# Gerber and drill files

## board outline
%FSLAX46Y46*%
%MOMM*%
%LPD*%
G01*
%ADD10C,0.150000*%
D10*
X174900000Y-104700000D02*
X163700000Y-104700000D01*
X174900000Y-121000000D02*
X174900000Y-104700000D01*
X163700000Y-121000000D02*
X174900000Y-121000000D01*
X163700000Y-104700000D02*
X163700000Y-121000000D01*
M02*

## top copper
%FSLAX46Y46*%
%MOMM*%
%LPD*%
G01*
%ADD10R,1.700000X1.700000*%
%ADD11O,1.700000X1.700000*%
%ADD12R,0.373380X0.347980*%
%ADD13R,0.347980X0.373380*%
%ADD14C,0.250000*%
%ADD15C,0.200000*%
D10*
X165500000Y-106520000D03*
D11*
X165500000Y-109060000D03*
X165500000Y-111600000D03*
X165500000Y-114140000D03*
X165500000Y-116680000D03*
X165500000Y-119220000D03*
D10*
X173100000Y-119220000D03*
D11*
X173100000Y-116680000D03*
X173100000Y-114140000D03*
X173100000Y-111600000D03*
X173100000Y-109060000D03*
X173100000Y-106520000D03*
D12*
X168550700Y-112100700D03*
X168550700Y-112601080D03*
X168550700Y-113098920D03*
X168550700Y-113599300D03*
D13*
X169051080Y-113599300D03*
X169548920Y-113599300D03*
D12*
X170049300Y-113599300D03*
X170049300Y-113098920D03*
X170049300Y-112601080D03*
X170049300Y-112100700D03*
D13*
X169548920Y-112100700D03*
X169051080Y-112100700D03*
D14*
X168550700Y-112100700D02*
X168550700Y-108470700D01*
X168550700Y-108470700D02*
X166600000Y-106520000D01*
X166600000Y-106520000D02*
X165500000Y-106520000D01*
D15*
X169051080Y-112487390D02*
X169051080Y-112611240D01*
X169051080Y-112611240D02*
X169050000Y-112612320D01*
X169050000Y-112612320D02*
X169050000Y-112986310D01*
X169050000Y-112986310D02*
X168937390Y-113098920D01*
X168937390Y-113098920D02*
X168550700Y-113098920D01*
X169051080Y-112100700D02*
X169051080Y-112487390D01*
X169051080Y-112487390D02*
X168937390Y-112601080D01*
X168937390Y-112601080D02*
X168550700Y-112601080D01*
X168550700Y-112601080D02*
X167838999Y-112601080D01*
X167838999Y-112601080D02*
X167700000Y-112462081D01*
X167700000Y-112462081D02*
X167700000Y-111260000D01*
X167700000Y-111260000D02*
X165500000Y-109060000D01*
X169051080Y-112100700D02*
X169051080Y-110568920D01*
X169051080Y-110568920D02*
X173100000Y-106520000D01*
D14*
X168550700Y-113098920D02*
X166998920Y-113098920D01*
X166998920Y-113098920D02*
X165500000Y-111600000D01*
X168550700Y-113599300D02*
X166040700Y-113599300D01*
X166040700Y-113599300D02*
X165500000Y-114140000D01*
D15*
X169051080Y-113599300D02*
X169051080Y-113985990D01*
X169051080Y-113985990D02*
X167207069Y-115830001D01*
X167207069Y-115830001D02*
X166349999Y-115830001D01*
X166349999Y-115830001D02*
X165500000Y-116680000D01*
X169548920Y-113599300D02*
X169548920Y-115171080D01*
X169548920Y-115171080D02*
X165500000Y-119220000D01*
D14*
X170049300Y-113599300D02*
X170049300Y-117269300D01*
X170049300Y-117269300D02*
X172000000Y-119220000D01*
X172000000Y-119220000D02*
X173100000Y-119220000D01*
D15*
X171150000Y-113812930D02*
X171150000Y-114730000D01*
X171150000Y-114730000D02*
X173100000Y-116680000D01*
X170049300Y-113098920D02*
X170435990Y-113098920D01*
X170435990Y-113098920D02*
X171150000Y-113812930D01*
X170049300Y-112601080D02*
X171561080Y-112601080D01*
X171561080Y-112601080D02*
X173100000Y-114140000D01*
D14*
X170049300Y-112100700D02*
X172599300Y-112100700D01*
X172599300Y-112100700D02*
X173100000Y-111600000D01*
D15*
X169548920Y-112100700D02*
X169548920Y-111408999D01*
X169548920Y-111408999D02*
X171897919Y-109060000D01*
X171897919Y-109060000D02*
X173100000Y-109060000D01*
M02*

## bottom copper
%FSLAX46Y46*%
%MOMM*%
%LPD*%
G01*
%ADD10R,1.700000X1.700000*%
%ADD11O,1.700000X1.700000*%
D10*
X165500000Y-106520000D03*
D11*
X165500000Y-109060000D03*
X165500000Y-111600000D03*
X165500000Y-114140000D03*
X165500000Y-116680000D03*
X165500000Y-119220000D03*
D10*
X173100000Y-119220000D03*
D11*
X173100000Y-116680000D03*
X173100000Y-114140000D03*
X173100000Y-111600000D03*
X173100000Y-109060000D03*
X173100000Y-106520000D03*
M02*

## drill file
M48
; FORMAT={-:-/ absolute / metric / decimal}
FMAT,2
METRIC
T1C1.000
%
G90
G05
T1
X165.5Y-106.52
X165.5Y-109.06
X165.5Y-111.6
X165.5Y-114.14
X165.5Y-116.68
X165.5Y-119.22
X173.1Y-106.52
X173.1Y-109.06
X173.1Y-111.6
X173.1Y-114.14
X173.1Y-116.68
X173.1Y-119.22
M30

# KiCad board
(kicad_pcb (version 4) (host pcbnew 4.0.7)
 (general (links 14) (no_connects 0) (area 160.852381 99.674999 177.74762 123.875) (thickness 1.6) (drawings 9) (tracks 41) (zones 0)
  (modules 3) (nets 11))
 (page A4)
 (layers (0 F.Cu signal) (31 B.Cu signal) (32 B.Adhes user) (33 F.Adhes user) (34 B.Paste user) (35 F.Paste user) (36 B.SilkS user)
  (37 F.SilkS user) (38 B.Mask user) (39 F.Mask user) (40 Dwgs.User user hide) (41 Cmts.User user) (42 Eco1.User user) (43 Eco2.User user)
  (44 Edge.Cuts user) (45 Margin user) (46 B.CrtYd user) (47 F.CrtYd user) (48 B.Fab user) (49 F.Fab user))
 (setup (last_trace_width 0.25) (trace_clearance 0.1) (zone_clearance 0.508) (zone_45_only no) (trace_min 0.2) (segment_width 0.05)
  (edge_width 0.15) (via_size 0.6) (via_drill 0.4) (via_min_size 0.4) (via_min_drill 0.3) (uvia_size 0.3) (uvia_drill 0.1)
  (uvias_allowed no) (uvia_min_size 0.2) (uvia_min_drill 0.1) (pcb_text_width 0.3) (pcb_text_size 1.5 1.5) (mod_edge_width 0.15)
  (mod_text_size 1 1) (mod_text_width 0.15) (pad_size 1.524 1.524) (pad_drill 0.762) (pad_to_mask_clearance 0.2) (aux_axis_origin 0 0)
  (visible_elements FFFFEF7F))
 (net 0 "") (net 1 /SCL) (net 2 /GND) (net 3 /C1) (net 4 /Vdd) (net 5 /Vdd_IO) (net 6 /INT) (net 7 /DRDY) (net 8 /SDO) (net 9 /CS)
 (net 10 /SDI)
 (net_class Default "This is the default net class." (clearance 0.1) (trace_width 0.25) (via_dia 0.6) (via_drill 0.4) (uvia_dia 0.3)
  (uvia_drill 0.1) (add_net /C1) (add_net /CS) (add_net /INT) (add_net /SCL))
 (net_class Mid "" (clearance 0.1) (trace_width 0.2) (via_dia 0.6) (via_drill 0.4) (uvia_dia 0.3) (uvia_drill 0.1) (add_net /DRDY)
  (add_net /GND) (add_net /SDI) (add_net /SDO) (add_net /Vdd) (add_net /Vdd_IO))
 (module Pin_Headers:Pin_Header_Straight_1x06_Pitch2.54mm (layer F.Cu) (at 165.5 106.52)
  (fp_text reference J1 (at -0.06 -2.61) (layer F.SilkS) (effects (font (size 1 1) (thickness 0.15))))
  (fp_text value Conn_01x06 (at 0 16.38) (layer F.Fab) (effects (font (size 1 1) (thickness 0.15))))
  (pad 1 thru_hole rect (at 0 0) (size 1.7 1.7) (drill 1) (layers *.Cu *.Mask) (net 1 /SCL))
  (pad 2 thru_hole oval (at 0 2.54) (size 1.7 1.7) (drill 1) (layers *.Cu *.Mask) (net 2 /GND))
  (pad 3 thru_hole oval (at 0 5.08) (size 1.7 1.7) (drill 1) (layers *.Cu *.Mask) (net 2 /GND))
  (pad 4 thru_hole oval (at 0 7.62) (size 1.7 1.7) (drill 1) (layers *.Cu *.Mask) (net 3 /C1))
  (pad 5 thru_hole oval (at 0 10.16) (size 1.7 1.7) (drill 1) (layers *.Cu *.Mask) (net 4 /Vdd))
  (pad 6 thru_hole oval (at 0 12.7) (size 1.7 1.7) (drill 1) (layers *.Cu *.Mask) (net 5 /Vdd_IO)))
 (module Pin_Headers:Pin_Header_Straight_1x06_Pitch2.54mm (layer F.Cu) (at 173.1 119.22 180)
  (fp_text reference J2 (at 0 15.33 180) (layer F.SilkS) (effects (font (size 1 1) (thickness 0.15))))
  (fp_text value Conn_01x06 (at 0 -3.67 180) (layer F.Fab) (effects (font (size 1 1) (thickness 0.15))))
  (pad 1 thru_hole rect (at 0 0 180) (size 1.7 1.7) (drill 1) (layers *.Cu *.Mask) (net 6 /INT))
  (pad 2 thru_hole oval (at 0 2.54 180) (size 1.7 1.7) (drill 1) (layers *.Cu *.Mask) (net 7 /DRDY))
  (pad 3 thru_hole oval (at 0 5.08 180) (size 1.7 1.7) (drill 1) (layers *.Cu *.Mask) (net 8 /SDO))
  (pad 4 thru_hole oval (at 0 7.62 180) (size 1.7 1.7) (drill 1) (layers *.Cu *.Mask) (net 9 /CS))
  (pad 5 thru_hole oval (at 0 10.16 180) (size 1.7 1.7) (drill 1) (layers *.Cu *.Mask) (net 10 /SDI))
  (pad 6 thru_hole oval (at 0 12.7 180) (size 1.7 1.7) (drill 1) (layers *.Cu *.Mask) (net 2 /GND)))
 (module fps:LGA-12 (layer F.Cu) (at 169.3 112.85)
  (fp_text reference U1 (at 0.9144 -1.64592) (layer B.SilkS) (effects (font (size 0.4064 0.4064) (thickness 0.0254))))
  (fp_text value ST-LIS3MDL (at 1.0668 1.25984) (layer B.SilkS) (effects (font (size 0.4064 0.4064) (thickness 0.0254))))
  (pad 1 smd rect (at -0.7493 -0.7493 90) (size 0.34798 0.37338) (layers F.Cu F.Paste F.Mask) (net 1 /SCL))
  (pad 2 smd rect (at -0.7493 -0.24892 90) (size 0.34798 0.37338) (layers F.Cu F.Paste F.Mask) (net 2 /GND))
  (pad 3 smd rect (at -0.7493 0.24892 90) (size 0.34798 0.37338) (layers F.Cu F.Paste F.Mask) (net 2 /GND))
  (pad 4 smd rect (at -0.7493 0.7493 90) (size 0.34798 0.37338) (layers F.Cu F.Paste F.Mask) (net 3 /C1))
  (pad 5 smd rect (at -0.24892 0.7493 180) (size 0.34798 0.37338) (layers F.Cu F.Paste F.Mask) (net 4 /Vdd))
  (pad 6 smd rect (at 0.24892 0.7493 180) (size 0.34798 0.37338) (layers F.Cu F.Paste F.Mask) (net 5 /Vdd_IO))
  (pad 7 smd rect (at 0.7493 0.7493 270) (size 0.34798 0.37338) (layers F.Cu F.Paste F.Mask) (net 6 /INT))
  (pad 8 smd rect (at 0.7493 0.24892 270) (size 0.34798 0.37338) (layers F.Cu F.Paste F.Mask) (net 7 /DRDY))
  (pad 9 smd rect (at 0.7493 -0.24892 270) (size 0.34798 0.37338) (layers F.Cu F.Paste F.Mask) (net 8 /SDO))
  (pad 10 smd rect (at 0.7493 -0.7493 270) (size 0.34798 0.37338) (layers F.Cu F.Paste F.Mask) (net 9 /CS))
  (pad 11 smd rect (at 0.24892 -0.7493) (size 0.34798 0.37338) (layers F.Cu F.Paste F.Mask) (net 10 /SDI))
  (pad 12 smd rect (at -0.24892 -0.7493) (size 0.34798 0.37338) (layers F.Cu F.Paste F.Mask) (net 2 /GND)))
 (gr_line (start 174.9 104.7) (end 163.7 104.7) (layer Edge.Cuts) (width 0.15))
 (gr_line (start 174.9 121) (end 174.9 104.7) (layer Edge.Cuts) (width 0.15))
 (gr_line (start 163.7 121) (end 174.9 121) (layer Edge.Cuts) (width 0.15))
 (gr_line (start 163.7 104.7) (end 163.7 121) (layer Edge.Cuts) (width 0.15))
 (segment (start 168.5507 112.1007) (end 168.5507 108.4707) (width 0.25) (layer F.Cu) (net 1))
 (segment (start 168.5507 108.4707) (end 166.6 106.52) (width 0.25) (layer F.Cu) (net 1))
 (segment (start 166.6 106.52) (end 165.5 106.52) (width 0.25) (layer F.Cu) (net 1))
 (segment (start 169.05108 112.48739) (end 169.05108 112.61124) (width 0.2) (layer F.Cu) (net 2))
 (segment (start 169.05108 112.61124) (end 169.05 112.61232) (width 0.2) (layer F.Cu) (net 2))
 (segment (start 169.05 112.61232) (end 169.05 112.98631) (width 0.2) (layer F.Cu) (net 2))
 (segment (start 169.05 112.98631) (end 168.93739 113.09892) (width 0.2) (layer F.Cu) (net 2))
 (segment (start 168.93739 113.09892) (end 168.5507 113.09892) (width 0.2) (layer F.Cu) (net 2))
 (segment (start 169.05108 112.1007) (end 169.05108 112.48739) (width 0.2) (layer F.Cu) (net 2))
 (segment (start 169.05108 112.48739) (end 168.93739 112.60108) (width 0.2) (layer F.Cu) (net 2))
 (segment (start 168.93739 112.60108) (end 168.5507 112.60108) (width 0.2) (layer F.Cu) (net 2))
 (segment (start 168.5507 112.60108) (end 167.838999 112.60108) (width 0.2) (layer F.Cu) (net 2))
 (segment (start 167.838999 112.60108) (end 167.7 112.462081) (width 0.2) (layer F.Cu) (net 2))
 (segment (start 167.7 112.462081) (end 167.7 111.26) (width 0.2) (layer F.Cu) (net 2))
 (segment (start 167.7 111.26) (end 165.5 109.06) (width 0.2) (layer F.Cu) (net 2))
 (segment (start 169.05108 112.1007) (end 169.05108 110.56892) (width 0.2) (layer F.Cu) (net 2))
 (segment (start 169.05108 110.56892) (end 173.1 106.52) (width 0.2) (layer F.Cu) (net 2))
 (segment (start 168.5507 113.09892) (end 166.99892 113.09892) (width 0.25) (layer F.Cu) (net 2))
 (segment (start 166.99892 113.09892) (end 165.5 111.6) (width 0.25) (layer F.Cu) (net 2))
 (segment (start 168.5507 113.5993) (end 166.0407 113.5993) (width 0.25) (layer F.Cu) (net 3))
 (segment (start 166.0407 113.5993) (end 165.5 114.14) (width 0.25) (layer F.Cu) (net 3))
 (segment (start 169.05108 113.5993) (end 169.05108 113.98599) (width 0.2) (layer F.Cu) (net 4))
 (segment (start 169.05108 113.98599) (end 167.207069 115.830001) (width 0.2) (layer F.Cu) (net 4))
 (segment (start 167.207069 115.830001) (end 166.349999 115.830001) (width 0.2) (layer F.Cu) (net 4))
 (segment (start 166.349999 115.830001) (end 165.5 116.68) (width 0.2) (layer F.Cu) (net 4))
 (segment (start 169.54892 113.5993) (end 169.54892 115.17108) (width 0.2) (layer F.Cu) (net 5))
 (segment (start 169.54892 115.17108) (end 165.5 119.22) (width 0.2) (layer F.Cu) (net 5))
 (segment (start 170.0493 113.5993) (end 170.0493 117.2693) (width 0.25) (layer F.Cu) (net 6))
 (segment (start 170.0493 117.2693) (end 172 119.22) (width 0.25) (layer F.Cu) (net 6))
 (segment (start 172 119.22) (end 173.1 119.22) (width 0.25) (layer F.Cu) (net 6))
 (segment (start 171.15 113.81293) (end 171.15 114.73) (width 0.2) (layer F.Cu) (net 7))
 (segment (start 171.15 114.73) (end 173.1 116.68) (width 0.2) (layer F.Cu) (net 7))
 (segment (start 170.0493 113.09892) (end 170.43599 113.09892) (width 0.2) (layer F.Cu) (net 7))
 (segment (start 170.43599 113.09892) (end 171.15 113.81293) (width 0.2) (layer F.Cu) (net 7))
 (segment (start 170.0493 112.60108) (end 171.56108 112.60108) (width 0.2) (layer F.Cu) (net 8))
 (segment (start 171.56108 112.60108) (end 173.1 114.14) (width 0.2) (layer F.Cu) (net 8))
 (segment (start 170.0493 112.1007) (end 172.5993 112.1007) (width 0.25) (layer F.Cu) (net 9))
 (segment (start 172.5993 112.1007) (end 173.1 111.6) (width 0.25) (layer F.Cu) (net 9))
 (segment (start 169.54892 112.1007) (end 169.54892 111.408999) (width 0.2) (layer F.Cu) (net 10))
 (segment (start 169.54892 111.408999) (end 171.897919 109.06) (width 0.2) (layer F.Cu) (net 10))
 (segment (start 171.897919 109.06) (end 173.1 109.06) (width 0.2) (layer F.Cu) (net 10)))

